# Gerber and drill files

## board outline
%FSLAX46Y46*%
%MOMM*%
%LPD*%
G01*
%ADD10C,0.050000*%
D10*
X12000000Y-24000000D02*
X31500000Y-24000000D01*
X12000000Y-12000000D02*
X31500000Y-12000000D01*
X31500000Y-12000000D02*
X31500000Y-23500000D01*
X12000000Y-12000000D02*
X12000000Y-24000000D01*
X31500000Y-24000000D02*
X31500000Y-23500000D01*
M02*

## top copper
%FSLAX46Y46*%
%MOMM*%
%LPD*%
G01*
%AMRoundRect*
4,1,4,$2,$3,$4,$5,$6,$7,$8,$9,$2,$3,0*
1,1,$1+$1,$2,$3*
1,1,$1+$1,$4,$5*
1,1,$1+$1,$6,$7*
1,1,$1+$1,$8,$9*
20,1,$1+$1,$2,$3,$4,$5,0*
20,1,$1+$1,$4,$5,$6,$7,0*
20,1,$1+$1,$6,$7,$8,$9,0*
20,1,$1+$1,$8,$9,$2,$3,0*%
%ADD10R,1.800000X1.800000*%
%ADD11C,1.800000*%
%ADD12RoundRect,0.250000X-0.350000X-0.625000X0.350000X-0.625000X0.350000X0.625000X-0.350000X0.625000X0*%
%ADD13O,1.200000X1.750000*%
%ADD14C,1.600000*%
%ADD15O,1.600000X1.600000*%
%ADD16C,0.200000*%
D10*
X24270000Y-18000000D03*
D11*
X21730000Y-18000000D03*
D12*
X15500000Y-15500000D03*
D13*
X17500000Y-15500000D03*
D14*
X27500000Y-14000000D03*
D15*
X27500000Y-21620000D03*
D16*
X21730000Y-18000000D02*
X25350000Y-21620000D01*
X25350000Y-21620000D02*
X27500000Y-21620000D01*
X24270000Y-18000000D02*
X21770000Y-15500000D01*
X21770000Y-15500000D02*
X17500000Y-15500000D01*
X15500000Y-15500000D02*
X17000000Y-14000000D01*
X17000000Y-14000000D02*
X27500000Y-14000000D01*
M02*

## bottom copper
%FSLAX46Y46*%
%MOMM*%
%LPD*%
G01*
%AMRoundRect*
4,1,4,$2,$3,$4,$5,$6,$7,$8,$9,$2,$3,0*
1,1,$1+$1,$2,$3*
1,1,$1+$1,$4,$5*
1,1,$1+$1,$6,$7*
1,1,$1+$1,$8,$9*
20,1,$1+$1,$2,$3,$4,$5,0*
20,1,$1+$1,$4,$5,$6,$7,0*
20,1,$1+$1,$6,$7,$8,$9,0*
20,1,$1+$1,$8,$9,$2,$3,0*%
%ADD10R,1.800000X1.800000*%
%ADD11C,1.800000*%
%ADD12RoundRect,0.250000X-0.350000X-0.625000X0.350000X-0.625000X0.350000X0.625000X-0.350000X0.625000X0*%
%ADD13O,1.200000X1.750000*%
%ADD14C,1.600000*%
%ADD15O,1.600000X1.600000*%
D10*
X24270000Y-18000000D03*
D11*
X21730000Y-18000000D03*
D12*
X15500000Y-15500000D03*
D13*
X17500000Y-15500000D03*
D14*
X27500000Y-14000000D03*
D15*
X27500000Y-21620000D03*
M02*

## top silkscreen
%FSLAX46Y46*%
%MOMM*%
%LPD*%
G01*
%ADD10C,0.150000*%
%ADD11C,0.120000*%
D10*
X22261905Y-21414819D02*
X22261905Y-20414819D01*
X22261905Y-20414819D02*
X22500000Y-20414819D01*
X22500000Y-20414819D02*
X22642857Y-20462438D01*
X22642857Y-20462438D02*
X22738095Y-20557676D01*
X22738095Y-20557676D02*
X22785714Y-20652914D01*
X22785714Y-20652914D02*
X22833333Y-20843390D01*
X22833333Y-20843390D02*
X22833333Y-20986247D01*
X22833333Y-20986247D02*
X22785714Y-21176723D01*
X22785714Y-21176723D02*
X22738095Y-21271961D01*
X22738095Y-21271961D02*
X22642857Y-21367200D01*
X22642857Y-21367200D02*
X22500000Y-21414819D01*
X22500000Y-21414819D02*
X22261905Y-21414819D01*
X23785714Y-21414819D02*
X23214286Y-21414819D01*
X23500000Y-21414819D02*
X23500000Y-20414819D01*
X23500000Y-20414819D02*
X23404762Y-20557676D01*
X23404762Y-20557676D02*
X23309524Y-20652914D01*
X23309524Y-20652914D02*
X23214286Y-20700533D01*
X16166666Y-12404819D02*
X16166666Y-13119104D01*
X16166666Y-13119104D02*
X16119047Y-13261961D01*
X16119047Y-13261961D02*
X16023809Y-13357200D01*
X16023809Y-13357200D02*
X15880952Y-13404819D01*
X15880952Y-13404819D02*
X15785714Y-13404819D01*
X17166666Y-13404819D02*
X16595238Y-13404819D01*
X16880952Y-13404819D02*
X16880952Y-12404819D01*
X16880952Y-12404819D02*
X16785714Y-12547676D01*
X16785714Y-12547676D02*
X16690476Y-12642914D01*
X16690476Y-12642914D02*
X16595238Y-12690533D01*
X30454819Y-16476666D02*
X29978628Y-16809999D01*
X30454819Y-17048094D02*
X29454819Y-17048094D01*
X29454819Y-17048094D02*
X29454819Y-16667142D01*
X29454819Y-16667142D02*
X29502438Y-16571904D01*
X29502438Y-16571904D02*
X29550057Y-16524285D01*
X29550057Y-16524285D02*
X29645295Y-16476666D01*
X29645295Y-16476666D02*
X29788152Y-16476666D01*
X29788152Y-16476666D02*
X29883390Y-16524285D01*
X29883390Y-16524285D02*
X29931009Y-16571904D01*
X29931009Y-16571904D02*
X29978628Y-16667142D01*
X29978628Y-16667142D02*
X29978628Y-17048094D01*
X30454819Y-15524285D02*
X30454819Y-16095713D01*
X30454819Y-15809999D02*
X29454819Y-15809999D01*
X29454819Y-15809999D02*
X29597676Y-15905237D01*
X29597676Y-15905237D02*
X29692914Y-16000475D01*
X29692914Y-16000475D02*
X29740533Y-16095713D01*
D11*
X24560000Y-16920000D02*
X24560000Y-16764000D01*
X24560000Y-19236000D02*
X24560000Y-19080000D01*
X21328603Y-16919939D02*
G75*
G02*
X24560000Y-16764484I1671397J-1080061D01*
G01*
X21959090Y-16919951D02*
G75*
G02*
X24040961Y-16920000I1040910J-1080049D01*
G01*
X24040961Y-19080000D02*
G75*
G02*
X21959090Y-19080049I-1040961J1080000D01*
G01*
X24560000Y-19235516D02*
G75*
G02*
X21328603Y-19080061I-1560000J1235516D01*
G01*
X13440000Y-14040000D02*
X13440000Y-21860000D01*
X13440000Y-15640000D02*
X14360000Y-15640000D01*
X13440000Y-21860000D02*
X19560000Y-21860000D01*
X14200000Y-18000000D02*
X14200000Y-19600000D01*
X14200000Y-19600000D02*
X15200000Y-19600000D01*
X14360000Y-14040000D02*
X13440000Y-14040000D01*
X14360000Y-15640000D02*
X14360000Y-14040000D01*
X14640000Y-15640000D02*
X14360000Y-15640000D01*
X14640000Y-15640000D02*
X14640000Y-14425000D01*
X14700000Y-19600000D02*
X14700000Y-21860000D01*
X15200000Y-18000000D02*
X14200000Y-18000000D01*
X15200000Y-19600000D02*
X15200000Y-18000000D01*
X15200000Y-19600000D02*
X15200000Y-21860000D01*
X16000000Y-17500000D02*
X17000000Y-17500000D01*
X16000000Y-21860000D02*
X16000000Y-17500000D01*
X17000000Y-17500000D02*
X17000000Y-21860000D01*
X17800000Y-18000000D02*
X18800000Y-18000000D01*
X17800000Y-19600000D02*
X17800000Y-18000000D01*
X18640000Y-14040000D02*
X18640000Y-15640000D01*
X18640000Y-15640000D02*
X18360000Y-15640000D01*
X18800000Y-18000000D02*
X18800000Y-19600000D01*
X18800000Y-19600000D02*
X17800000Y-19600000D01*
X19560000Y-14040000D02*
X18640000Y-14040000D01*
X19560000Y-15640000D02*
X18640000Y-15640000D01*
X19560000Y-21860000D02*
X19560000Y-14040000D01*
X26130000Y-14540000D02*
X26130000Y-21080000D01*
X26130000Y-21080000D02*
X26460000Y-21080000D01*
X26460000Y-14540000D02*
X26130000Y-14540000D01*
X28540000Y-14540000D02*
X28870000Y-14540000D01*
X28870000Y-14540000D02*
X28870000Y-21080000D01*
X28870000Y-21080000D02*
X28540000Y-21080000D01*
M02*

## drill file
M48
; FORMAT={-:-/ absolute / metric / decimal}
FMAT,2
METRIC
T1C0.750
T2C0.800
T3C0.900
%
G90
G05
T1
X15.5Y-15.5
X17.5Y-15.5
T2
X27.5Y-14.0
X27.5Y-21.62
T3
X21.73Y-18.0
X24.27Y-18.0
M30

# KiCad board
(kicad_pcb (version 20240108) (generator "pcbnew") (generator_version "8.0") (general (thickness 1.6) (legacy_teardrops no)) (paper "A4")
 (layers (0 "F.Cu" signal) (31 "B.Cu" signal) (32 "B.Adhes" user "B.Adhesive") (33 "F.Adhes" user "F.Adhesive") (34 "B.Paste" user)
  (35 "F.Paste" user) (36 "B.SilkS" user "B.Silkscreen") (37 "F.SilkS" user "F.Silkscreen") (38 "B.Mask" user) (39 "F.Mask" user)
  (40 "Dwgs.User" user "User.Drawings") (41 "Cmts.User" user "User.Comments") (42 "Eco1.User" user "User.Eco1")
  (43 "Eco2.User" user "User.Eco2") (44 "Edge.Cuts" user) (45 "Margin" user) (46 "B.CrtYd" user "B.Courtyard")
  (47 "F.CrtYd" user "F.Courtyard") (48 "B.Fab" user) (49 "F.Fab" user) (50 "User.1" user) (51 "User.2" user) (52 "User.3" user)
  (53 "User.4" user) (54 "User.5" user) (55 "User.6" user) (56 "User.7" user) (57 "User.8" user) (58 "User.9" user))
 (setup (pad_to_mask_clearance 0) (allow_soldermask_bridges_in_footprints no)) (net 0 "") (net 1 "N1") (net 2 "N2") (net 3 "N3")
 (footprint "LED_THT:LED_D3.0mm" (layer "F.Cu") (at 24.27 18 180)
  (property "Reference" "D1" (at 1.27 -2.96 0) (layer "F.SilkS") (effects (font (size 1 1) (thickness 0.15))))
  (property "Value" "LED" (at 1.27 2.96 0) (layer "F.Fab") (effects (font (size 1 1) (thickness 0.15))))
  (fp_line (start -0.29 1.08) (end -0.29 1.236) (stroke (width 0.12) (type solid)) (layer "F.SilkS"))
  (fp_line (start -0.29 -1.236) (end -0.29 -1.08) (stroke (width 0.12) (type solid)) (layer "F.SilkS"))
  (fp_arc (start 2.941397 1.080061) (mid 1.365624 1.987701) (end -0.29 1.235516) (stroke (width 0.12) (type solid)) (layer "F.SilkS"))
  (fp_arc (start 2.31091 1.080049) (mid 1.269965 1.5) (end 0.229039 1.08) (stroke (width 0.12) (type solid)) (layer "F.SilkS"))
  (fp_arc (start 0.229039 -1.08) (mid 1.269965 -1.5) (end 2.31091 -1.080049) (stroke (width 0.12) (type solid)) (layer "F.SilkS"))
  (fp_arc (start -0.29 -1.235516) (mid 1.365624 -1.987701) (end 2.941397 -1.080061) (stroke (width 0.12) (type solid)) (layer "F.SilkS"))
  (pad "1" thru_hole rect (at 0 0 180) (size 1.8 1.8) (drill 0.9) (layers "*.Cu" "*.Mask") (remove_unused_layers no) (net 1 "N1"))
  (pad "2" thru_hole circle (at 2.54 0 180) (size 1.8 1.8) (drill 0.9) (layers "*.Cu" "*.Mask") (remove_unused_layers no) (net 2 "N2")))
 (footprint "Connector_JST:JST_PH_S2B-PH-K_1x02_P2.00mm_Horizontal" (layer "F.Cu") (at 15.5 15.5)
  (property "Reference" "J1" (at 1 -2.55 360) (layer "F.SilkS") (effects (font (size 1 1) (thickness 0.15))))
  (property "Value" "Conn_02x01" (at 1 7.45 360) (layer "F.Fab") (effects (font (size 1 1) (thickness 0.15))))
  (fp_line (start -2.06 -1.46) (end -2.06 6.36) (stroke (width 0.12) (type solid)) (layer "F.SilkS"))
  (fp_line (start -2.06 0.14) (end -1.14 0.14) (stroke (width 0.12) (type solid)) (layer "F.SilkS"))
  (fp_line (start -2.06 6.36) (end 4.06 6.36) (stroke (width 0.12) (type solid)) (layer "F.SilkS"))
  (fp_line (start -1.3 2.5) (end -1.3 4.1) (stroke (width 0.12) (type solid)) (layer "F.SilkS"))
  (fp_line (start -1.3 4.1) (end -0.3 4.1) (stroke (width 0.12) (type solid)) (layer "F.SilkS"))
  (fp_line (start -1.14 -1.46) (end -2.06 -1.46) (stroke (width 0.12) (type solid)) (layer "F.SilkS"))
  (fp_line (start -1.14 0.14) (end -1.14 -1.46) (stroke (width 0.12) (type solid)) (layer "F.SilkS"))
  (fp_line (start -0.86 0.14) (end -1.14 0.14) (stroke (width 0.12) (type solid)) (layer "F.SilkS"))
  (fp_line (start -0.86 0.14) (end -0.86 -1.075) (stroke (width 0.12) (type solid)) (layer "F.SilkS"))
  (fp_line (start -0.8 4.1) (end -0.8 6.36) (stroke (width 0.12) (type solid)) (layer "F.SilkS"))
  (fp_line (start -0.3 2.5) (end -1.3 2.5) (stroke (width 0.12) (type solid)) (layer "F.SilkS"))
  (fp_line (start -0.3 4.1) (end -0.3 2.5) (stroke (width 0.12) (type solid)) (layer "F.SilkS"))
  (fp_line (start -0.3 4.1) (end -0.3 6.36) (stroke (width 0.12) (type solid)) (layer "F.SilkS"))
  (fp_line (start 0.5 2) (end 1.5 2) (stroke (width 0.12) (type solid)) (layer "F.SilkS"))
  (fp_line (start 0.5 6.36) (end 0.5 2) (stroke (width 0.12) (type solid)) (layer "F.SilkS"))
  (fp_line (start 1.5 2) (end 1.5 6.36) (stroke (width 0.12) (type solid)) (layer "F.SilkS"))
  (fp_line (start 2.3 2.5) (end 3.3 2.5) (stroke (width 0.12) (type solid)) (layer "F.SilkS"))
  (fp_line (start 2.3 4.1) (end 2.3 2.5) (stroke (width 0.12) (type solid)) (layer "F.SilkS"))
  (fp_line (start 3.14 -1.46) (end 3.14 0.14) (stroke (width 0.12) (type solid)) (layer "F.SilkS"))
  (fp_line (start 3.14 0.14) (end 2.86 0.14) (stroke (width 0.12) (type solid)) (layer "F.SilkS"))
  (fp_line (start 3.3 2.5) (end 3.3 4.1) (stroke (width 0.12) (type solid)) (layer "F.SilkS"))
  (fp_line (start 3.3 4.1) (end 2.3 4.1) (stroke (width 0.12) (type solid)) (layer "F.SilkS"))
  (fp_line (start 4.06 -1.46) (end 3.14 -1.46) (stroke (width 0.12) (type solid)) (layer "F.SilkS"))
  (fp_line (start 4.06 0.14) (end 3.14 0.14) (stroke (width 0.12) (type solid)) (layer "F.SilkS"))
  (fp_line (start 4.06 6.36) (end 4.06 -1.46) (stroke (width 0.12) (type solid)) (layer "F.SilkS"))
  (pad "1" thru_hole roundrect (at 0 0) (size 1.2 1.75) (drill 0.75) (layers "*.Cu" "*.Mask") (remove_unused_layers no)
   (roundrect_rratio 0.208333) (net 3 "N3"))
  (pad "2" thru_hole oval (at 2 0) (size 1.2 1.75) (drill 0.75) (layers "*.Cu" "*.Mask") (remove_unused_layers no) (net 1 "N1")))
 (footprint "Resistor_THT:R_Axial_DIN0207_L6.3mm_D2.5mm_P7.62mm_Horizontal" (layer "F.Cu") (at 27.5 14 -90)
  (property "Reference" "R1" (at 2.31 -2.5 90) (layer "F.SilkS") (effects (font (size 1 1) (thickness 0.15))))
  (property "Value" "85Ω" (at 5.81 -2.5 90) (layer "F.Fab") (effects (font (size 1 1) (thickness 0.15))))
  (fp_line (start 0.54 1.37) (end 7.08 1.37) (stroke (width 0.12) (type solid)) (layer "F.SilkS"))
  (fp_line (start 7.08 1.37) (end 7.08 1.04) (stroke (width 0.12) (type solid)) (layer "F.SilkS"))
  (fp_line (start 0.54 1.04) (end 0.54 1.37) (stroke (width 0.12) (type solid)) (layer "F.SilkS"))
  (fp_line (start 0.54 -1.04) (end 0.54 -1.37) (stroke (width 0.12) (type solid)) (layer "F.SilkS"))
  (fp_line (start 0.54 -1.37) (end 7.08 -1.37) (stroke (width 0.12) (type solid)) (layer "F.SilkS"))
  (fp_line (start 7.08 -1.37) (end 7.08 -1.04) (stroke (width 0.12) (type solid)) (layer "F.SilkS"))
  (pad "1" thru_hole circle (at 0 0 270) (size 1.6 1.6) (drill 0.8) (layers "*.Cu" "*.Mask") (remove_unused_layers no) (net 3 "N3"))
  (pad "2" thru_hole oval (at 7.62 0 270) (size 1.6 1.6) (drill 0.8) (layers "*.Cu" "*.Mask") (remove_unused_layers no) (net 2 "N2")))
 (gr_line (start 12 24) (end 31.5 24) (stroke (width 0.05) (type default)) (layer "Edge.Cuts"))
 (gr_line (start 12 12) (end 31.5 12) (stroke (width 0.05) (type default)) (layer "Edge.Cuts"))
 (gr_line (start 31.5 12) (end 31.5 23.5) (stroke (width 0.05) (type default)) (layer "Edge.Cuts"))
 (gr_line (start 12 12) (end 12 24) (stroke (width 0.05) (type default)) (layer "Edge.Cuts"))
 (gr_line (start 31.5 24) (end 31.5 23.5) (stroke (width 0.05) (type default)) (layer "Edge.Cuts"))
 (segment (start 21.73 18) (end 25.35 21.62) (width 0.2) (layer "F.Cu") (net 2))
 (segment (start 25.35 21.62) (end 27.5 21.62) (width 0.2) (layer "F.Cu") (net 2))
 (segment (start 24.27 18) (end 21.77 15.5) (width 0.2) (layer "F.Cu") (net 1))
 (segment (start 21.77 15.5) (end 17.5 15.5) (width 0.2) (layer "F.Cu") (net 1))
 (segment (start 15.5 15.5) (end 17 14) (width 0.2) (layer "F.Cu") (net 3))
 (segment (start 17 14) (end 27.5 14) (width 0.2) (layer "F.Cu") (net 3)))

